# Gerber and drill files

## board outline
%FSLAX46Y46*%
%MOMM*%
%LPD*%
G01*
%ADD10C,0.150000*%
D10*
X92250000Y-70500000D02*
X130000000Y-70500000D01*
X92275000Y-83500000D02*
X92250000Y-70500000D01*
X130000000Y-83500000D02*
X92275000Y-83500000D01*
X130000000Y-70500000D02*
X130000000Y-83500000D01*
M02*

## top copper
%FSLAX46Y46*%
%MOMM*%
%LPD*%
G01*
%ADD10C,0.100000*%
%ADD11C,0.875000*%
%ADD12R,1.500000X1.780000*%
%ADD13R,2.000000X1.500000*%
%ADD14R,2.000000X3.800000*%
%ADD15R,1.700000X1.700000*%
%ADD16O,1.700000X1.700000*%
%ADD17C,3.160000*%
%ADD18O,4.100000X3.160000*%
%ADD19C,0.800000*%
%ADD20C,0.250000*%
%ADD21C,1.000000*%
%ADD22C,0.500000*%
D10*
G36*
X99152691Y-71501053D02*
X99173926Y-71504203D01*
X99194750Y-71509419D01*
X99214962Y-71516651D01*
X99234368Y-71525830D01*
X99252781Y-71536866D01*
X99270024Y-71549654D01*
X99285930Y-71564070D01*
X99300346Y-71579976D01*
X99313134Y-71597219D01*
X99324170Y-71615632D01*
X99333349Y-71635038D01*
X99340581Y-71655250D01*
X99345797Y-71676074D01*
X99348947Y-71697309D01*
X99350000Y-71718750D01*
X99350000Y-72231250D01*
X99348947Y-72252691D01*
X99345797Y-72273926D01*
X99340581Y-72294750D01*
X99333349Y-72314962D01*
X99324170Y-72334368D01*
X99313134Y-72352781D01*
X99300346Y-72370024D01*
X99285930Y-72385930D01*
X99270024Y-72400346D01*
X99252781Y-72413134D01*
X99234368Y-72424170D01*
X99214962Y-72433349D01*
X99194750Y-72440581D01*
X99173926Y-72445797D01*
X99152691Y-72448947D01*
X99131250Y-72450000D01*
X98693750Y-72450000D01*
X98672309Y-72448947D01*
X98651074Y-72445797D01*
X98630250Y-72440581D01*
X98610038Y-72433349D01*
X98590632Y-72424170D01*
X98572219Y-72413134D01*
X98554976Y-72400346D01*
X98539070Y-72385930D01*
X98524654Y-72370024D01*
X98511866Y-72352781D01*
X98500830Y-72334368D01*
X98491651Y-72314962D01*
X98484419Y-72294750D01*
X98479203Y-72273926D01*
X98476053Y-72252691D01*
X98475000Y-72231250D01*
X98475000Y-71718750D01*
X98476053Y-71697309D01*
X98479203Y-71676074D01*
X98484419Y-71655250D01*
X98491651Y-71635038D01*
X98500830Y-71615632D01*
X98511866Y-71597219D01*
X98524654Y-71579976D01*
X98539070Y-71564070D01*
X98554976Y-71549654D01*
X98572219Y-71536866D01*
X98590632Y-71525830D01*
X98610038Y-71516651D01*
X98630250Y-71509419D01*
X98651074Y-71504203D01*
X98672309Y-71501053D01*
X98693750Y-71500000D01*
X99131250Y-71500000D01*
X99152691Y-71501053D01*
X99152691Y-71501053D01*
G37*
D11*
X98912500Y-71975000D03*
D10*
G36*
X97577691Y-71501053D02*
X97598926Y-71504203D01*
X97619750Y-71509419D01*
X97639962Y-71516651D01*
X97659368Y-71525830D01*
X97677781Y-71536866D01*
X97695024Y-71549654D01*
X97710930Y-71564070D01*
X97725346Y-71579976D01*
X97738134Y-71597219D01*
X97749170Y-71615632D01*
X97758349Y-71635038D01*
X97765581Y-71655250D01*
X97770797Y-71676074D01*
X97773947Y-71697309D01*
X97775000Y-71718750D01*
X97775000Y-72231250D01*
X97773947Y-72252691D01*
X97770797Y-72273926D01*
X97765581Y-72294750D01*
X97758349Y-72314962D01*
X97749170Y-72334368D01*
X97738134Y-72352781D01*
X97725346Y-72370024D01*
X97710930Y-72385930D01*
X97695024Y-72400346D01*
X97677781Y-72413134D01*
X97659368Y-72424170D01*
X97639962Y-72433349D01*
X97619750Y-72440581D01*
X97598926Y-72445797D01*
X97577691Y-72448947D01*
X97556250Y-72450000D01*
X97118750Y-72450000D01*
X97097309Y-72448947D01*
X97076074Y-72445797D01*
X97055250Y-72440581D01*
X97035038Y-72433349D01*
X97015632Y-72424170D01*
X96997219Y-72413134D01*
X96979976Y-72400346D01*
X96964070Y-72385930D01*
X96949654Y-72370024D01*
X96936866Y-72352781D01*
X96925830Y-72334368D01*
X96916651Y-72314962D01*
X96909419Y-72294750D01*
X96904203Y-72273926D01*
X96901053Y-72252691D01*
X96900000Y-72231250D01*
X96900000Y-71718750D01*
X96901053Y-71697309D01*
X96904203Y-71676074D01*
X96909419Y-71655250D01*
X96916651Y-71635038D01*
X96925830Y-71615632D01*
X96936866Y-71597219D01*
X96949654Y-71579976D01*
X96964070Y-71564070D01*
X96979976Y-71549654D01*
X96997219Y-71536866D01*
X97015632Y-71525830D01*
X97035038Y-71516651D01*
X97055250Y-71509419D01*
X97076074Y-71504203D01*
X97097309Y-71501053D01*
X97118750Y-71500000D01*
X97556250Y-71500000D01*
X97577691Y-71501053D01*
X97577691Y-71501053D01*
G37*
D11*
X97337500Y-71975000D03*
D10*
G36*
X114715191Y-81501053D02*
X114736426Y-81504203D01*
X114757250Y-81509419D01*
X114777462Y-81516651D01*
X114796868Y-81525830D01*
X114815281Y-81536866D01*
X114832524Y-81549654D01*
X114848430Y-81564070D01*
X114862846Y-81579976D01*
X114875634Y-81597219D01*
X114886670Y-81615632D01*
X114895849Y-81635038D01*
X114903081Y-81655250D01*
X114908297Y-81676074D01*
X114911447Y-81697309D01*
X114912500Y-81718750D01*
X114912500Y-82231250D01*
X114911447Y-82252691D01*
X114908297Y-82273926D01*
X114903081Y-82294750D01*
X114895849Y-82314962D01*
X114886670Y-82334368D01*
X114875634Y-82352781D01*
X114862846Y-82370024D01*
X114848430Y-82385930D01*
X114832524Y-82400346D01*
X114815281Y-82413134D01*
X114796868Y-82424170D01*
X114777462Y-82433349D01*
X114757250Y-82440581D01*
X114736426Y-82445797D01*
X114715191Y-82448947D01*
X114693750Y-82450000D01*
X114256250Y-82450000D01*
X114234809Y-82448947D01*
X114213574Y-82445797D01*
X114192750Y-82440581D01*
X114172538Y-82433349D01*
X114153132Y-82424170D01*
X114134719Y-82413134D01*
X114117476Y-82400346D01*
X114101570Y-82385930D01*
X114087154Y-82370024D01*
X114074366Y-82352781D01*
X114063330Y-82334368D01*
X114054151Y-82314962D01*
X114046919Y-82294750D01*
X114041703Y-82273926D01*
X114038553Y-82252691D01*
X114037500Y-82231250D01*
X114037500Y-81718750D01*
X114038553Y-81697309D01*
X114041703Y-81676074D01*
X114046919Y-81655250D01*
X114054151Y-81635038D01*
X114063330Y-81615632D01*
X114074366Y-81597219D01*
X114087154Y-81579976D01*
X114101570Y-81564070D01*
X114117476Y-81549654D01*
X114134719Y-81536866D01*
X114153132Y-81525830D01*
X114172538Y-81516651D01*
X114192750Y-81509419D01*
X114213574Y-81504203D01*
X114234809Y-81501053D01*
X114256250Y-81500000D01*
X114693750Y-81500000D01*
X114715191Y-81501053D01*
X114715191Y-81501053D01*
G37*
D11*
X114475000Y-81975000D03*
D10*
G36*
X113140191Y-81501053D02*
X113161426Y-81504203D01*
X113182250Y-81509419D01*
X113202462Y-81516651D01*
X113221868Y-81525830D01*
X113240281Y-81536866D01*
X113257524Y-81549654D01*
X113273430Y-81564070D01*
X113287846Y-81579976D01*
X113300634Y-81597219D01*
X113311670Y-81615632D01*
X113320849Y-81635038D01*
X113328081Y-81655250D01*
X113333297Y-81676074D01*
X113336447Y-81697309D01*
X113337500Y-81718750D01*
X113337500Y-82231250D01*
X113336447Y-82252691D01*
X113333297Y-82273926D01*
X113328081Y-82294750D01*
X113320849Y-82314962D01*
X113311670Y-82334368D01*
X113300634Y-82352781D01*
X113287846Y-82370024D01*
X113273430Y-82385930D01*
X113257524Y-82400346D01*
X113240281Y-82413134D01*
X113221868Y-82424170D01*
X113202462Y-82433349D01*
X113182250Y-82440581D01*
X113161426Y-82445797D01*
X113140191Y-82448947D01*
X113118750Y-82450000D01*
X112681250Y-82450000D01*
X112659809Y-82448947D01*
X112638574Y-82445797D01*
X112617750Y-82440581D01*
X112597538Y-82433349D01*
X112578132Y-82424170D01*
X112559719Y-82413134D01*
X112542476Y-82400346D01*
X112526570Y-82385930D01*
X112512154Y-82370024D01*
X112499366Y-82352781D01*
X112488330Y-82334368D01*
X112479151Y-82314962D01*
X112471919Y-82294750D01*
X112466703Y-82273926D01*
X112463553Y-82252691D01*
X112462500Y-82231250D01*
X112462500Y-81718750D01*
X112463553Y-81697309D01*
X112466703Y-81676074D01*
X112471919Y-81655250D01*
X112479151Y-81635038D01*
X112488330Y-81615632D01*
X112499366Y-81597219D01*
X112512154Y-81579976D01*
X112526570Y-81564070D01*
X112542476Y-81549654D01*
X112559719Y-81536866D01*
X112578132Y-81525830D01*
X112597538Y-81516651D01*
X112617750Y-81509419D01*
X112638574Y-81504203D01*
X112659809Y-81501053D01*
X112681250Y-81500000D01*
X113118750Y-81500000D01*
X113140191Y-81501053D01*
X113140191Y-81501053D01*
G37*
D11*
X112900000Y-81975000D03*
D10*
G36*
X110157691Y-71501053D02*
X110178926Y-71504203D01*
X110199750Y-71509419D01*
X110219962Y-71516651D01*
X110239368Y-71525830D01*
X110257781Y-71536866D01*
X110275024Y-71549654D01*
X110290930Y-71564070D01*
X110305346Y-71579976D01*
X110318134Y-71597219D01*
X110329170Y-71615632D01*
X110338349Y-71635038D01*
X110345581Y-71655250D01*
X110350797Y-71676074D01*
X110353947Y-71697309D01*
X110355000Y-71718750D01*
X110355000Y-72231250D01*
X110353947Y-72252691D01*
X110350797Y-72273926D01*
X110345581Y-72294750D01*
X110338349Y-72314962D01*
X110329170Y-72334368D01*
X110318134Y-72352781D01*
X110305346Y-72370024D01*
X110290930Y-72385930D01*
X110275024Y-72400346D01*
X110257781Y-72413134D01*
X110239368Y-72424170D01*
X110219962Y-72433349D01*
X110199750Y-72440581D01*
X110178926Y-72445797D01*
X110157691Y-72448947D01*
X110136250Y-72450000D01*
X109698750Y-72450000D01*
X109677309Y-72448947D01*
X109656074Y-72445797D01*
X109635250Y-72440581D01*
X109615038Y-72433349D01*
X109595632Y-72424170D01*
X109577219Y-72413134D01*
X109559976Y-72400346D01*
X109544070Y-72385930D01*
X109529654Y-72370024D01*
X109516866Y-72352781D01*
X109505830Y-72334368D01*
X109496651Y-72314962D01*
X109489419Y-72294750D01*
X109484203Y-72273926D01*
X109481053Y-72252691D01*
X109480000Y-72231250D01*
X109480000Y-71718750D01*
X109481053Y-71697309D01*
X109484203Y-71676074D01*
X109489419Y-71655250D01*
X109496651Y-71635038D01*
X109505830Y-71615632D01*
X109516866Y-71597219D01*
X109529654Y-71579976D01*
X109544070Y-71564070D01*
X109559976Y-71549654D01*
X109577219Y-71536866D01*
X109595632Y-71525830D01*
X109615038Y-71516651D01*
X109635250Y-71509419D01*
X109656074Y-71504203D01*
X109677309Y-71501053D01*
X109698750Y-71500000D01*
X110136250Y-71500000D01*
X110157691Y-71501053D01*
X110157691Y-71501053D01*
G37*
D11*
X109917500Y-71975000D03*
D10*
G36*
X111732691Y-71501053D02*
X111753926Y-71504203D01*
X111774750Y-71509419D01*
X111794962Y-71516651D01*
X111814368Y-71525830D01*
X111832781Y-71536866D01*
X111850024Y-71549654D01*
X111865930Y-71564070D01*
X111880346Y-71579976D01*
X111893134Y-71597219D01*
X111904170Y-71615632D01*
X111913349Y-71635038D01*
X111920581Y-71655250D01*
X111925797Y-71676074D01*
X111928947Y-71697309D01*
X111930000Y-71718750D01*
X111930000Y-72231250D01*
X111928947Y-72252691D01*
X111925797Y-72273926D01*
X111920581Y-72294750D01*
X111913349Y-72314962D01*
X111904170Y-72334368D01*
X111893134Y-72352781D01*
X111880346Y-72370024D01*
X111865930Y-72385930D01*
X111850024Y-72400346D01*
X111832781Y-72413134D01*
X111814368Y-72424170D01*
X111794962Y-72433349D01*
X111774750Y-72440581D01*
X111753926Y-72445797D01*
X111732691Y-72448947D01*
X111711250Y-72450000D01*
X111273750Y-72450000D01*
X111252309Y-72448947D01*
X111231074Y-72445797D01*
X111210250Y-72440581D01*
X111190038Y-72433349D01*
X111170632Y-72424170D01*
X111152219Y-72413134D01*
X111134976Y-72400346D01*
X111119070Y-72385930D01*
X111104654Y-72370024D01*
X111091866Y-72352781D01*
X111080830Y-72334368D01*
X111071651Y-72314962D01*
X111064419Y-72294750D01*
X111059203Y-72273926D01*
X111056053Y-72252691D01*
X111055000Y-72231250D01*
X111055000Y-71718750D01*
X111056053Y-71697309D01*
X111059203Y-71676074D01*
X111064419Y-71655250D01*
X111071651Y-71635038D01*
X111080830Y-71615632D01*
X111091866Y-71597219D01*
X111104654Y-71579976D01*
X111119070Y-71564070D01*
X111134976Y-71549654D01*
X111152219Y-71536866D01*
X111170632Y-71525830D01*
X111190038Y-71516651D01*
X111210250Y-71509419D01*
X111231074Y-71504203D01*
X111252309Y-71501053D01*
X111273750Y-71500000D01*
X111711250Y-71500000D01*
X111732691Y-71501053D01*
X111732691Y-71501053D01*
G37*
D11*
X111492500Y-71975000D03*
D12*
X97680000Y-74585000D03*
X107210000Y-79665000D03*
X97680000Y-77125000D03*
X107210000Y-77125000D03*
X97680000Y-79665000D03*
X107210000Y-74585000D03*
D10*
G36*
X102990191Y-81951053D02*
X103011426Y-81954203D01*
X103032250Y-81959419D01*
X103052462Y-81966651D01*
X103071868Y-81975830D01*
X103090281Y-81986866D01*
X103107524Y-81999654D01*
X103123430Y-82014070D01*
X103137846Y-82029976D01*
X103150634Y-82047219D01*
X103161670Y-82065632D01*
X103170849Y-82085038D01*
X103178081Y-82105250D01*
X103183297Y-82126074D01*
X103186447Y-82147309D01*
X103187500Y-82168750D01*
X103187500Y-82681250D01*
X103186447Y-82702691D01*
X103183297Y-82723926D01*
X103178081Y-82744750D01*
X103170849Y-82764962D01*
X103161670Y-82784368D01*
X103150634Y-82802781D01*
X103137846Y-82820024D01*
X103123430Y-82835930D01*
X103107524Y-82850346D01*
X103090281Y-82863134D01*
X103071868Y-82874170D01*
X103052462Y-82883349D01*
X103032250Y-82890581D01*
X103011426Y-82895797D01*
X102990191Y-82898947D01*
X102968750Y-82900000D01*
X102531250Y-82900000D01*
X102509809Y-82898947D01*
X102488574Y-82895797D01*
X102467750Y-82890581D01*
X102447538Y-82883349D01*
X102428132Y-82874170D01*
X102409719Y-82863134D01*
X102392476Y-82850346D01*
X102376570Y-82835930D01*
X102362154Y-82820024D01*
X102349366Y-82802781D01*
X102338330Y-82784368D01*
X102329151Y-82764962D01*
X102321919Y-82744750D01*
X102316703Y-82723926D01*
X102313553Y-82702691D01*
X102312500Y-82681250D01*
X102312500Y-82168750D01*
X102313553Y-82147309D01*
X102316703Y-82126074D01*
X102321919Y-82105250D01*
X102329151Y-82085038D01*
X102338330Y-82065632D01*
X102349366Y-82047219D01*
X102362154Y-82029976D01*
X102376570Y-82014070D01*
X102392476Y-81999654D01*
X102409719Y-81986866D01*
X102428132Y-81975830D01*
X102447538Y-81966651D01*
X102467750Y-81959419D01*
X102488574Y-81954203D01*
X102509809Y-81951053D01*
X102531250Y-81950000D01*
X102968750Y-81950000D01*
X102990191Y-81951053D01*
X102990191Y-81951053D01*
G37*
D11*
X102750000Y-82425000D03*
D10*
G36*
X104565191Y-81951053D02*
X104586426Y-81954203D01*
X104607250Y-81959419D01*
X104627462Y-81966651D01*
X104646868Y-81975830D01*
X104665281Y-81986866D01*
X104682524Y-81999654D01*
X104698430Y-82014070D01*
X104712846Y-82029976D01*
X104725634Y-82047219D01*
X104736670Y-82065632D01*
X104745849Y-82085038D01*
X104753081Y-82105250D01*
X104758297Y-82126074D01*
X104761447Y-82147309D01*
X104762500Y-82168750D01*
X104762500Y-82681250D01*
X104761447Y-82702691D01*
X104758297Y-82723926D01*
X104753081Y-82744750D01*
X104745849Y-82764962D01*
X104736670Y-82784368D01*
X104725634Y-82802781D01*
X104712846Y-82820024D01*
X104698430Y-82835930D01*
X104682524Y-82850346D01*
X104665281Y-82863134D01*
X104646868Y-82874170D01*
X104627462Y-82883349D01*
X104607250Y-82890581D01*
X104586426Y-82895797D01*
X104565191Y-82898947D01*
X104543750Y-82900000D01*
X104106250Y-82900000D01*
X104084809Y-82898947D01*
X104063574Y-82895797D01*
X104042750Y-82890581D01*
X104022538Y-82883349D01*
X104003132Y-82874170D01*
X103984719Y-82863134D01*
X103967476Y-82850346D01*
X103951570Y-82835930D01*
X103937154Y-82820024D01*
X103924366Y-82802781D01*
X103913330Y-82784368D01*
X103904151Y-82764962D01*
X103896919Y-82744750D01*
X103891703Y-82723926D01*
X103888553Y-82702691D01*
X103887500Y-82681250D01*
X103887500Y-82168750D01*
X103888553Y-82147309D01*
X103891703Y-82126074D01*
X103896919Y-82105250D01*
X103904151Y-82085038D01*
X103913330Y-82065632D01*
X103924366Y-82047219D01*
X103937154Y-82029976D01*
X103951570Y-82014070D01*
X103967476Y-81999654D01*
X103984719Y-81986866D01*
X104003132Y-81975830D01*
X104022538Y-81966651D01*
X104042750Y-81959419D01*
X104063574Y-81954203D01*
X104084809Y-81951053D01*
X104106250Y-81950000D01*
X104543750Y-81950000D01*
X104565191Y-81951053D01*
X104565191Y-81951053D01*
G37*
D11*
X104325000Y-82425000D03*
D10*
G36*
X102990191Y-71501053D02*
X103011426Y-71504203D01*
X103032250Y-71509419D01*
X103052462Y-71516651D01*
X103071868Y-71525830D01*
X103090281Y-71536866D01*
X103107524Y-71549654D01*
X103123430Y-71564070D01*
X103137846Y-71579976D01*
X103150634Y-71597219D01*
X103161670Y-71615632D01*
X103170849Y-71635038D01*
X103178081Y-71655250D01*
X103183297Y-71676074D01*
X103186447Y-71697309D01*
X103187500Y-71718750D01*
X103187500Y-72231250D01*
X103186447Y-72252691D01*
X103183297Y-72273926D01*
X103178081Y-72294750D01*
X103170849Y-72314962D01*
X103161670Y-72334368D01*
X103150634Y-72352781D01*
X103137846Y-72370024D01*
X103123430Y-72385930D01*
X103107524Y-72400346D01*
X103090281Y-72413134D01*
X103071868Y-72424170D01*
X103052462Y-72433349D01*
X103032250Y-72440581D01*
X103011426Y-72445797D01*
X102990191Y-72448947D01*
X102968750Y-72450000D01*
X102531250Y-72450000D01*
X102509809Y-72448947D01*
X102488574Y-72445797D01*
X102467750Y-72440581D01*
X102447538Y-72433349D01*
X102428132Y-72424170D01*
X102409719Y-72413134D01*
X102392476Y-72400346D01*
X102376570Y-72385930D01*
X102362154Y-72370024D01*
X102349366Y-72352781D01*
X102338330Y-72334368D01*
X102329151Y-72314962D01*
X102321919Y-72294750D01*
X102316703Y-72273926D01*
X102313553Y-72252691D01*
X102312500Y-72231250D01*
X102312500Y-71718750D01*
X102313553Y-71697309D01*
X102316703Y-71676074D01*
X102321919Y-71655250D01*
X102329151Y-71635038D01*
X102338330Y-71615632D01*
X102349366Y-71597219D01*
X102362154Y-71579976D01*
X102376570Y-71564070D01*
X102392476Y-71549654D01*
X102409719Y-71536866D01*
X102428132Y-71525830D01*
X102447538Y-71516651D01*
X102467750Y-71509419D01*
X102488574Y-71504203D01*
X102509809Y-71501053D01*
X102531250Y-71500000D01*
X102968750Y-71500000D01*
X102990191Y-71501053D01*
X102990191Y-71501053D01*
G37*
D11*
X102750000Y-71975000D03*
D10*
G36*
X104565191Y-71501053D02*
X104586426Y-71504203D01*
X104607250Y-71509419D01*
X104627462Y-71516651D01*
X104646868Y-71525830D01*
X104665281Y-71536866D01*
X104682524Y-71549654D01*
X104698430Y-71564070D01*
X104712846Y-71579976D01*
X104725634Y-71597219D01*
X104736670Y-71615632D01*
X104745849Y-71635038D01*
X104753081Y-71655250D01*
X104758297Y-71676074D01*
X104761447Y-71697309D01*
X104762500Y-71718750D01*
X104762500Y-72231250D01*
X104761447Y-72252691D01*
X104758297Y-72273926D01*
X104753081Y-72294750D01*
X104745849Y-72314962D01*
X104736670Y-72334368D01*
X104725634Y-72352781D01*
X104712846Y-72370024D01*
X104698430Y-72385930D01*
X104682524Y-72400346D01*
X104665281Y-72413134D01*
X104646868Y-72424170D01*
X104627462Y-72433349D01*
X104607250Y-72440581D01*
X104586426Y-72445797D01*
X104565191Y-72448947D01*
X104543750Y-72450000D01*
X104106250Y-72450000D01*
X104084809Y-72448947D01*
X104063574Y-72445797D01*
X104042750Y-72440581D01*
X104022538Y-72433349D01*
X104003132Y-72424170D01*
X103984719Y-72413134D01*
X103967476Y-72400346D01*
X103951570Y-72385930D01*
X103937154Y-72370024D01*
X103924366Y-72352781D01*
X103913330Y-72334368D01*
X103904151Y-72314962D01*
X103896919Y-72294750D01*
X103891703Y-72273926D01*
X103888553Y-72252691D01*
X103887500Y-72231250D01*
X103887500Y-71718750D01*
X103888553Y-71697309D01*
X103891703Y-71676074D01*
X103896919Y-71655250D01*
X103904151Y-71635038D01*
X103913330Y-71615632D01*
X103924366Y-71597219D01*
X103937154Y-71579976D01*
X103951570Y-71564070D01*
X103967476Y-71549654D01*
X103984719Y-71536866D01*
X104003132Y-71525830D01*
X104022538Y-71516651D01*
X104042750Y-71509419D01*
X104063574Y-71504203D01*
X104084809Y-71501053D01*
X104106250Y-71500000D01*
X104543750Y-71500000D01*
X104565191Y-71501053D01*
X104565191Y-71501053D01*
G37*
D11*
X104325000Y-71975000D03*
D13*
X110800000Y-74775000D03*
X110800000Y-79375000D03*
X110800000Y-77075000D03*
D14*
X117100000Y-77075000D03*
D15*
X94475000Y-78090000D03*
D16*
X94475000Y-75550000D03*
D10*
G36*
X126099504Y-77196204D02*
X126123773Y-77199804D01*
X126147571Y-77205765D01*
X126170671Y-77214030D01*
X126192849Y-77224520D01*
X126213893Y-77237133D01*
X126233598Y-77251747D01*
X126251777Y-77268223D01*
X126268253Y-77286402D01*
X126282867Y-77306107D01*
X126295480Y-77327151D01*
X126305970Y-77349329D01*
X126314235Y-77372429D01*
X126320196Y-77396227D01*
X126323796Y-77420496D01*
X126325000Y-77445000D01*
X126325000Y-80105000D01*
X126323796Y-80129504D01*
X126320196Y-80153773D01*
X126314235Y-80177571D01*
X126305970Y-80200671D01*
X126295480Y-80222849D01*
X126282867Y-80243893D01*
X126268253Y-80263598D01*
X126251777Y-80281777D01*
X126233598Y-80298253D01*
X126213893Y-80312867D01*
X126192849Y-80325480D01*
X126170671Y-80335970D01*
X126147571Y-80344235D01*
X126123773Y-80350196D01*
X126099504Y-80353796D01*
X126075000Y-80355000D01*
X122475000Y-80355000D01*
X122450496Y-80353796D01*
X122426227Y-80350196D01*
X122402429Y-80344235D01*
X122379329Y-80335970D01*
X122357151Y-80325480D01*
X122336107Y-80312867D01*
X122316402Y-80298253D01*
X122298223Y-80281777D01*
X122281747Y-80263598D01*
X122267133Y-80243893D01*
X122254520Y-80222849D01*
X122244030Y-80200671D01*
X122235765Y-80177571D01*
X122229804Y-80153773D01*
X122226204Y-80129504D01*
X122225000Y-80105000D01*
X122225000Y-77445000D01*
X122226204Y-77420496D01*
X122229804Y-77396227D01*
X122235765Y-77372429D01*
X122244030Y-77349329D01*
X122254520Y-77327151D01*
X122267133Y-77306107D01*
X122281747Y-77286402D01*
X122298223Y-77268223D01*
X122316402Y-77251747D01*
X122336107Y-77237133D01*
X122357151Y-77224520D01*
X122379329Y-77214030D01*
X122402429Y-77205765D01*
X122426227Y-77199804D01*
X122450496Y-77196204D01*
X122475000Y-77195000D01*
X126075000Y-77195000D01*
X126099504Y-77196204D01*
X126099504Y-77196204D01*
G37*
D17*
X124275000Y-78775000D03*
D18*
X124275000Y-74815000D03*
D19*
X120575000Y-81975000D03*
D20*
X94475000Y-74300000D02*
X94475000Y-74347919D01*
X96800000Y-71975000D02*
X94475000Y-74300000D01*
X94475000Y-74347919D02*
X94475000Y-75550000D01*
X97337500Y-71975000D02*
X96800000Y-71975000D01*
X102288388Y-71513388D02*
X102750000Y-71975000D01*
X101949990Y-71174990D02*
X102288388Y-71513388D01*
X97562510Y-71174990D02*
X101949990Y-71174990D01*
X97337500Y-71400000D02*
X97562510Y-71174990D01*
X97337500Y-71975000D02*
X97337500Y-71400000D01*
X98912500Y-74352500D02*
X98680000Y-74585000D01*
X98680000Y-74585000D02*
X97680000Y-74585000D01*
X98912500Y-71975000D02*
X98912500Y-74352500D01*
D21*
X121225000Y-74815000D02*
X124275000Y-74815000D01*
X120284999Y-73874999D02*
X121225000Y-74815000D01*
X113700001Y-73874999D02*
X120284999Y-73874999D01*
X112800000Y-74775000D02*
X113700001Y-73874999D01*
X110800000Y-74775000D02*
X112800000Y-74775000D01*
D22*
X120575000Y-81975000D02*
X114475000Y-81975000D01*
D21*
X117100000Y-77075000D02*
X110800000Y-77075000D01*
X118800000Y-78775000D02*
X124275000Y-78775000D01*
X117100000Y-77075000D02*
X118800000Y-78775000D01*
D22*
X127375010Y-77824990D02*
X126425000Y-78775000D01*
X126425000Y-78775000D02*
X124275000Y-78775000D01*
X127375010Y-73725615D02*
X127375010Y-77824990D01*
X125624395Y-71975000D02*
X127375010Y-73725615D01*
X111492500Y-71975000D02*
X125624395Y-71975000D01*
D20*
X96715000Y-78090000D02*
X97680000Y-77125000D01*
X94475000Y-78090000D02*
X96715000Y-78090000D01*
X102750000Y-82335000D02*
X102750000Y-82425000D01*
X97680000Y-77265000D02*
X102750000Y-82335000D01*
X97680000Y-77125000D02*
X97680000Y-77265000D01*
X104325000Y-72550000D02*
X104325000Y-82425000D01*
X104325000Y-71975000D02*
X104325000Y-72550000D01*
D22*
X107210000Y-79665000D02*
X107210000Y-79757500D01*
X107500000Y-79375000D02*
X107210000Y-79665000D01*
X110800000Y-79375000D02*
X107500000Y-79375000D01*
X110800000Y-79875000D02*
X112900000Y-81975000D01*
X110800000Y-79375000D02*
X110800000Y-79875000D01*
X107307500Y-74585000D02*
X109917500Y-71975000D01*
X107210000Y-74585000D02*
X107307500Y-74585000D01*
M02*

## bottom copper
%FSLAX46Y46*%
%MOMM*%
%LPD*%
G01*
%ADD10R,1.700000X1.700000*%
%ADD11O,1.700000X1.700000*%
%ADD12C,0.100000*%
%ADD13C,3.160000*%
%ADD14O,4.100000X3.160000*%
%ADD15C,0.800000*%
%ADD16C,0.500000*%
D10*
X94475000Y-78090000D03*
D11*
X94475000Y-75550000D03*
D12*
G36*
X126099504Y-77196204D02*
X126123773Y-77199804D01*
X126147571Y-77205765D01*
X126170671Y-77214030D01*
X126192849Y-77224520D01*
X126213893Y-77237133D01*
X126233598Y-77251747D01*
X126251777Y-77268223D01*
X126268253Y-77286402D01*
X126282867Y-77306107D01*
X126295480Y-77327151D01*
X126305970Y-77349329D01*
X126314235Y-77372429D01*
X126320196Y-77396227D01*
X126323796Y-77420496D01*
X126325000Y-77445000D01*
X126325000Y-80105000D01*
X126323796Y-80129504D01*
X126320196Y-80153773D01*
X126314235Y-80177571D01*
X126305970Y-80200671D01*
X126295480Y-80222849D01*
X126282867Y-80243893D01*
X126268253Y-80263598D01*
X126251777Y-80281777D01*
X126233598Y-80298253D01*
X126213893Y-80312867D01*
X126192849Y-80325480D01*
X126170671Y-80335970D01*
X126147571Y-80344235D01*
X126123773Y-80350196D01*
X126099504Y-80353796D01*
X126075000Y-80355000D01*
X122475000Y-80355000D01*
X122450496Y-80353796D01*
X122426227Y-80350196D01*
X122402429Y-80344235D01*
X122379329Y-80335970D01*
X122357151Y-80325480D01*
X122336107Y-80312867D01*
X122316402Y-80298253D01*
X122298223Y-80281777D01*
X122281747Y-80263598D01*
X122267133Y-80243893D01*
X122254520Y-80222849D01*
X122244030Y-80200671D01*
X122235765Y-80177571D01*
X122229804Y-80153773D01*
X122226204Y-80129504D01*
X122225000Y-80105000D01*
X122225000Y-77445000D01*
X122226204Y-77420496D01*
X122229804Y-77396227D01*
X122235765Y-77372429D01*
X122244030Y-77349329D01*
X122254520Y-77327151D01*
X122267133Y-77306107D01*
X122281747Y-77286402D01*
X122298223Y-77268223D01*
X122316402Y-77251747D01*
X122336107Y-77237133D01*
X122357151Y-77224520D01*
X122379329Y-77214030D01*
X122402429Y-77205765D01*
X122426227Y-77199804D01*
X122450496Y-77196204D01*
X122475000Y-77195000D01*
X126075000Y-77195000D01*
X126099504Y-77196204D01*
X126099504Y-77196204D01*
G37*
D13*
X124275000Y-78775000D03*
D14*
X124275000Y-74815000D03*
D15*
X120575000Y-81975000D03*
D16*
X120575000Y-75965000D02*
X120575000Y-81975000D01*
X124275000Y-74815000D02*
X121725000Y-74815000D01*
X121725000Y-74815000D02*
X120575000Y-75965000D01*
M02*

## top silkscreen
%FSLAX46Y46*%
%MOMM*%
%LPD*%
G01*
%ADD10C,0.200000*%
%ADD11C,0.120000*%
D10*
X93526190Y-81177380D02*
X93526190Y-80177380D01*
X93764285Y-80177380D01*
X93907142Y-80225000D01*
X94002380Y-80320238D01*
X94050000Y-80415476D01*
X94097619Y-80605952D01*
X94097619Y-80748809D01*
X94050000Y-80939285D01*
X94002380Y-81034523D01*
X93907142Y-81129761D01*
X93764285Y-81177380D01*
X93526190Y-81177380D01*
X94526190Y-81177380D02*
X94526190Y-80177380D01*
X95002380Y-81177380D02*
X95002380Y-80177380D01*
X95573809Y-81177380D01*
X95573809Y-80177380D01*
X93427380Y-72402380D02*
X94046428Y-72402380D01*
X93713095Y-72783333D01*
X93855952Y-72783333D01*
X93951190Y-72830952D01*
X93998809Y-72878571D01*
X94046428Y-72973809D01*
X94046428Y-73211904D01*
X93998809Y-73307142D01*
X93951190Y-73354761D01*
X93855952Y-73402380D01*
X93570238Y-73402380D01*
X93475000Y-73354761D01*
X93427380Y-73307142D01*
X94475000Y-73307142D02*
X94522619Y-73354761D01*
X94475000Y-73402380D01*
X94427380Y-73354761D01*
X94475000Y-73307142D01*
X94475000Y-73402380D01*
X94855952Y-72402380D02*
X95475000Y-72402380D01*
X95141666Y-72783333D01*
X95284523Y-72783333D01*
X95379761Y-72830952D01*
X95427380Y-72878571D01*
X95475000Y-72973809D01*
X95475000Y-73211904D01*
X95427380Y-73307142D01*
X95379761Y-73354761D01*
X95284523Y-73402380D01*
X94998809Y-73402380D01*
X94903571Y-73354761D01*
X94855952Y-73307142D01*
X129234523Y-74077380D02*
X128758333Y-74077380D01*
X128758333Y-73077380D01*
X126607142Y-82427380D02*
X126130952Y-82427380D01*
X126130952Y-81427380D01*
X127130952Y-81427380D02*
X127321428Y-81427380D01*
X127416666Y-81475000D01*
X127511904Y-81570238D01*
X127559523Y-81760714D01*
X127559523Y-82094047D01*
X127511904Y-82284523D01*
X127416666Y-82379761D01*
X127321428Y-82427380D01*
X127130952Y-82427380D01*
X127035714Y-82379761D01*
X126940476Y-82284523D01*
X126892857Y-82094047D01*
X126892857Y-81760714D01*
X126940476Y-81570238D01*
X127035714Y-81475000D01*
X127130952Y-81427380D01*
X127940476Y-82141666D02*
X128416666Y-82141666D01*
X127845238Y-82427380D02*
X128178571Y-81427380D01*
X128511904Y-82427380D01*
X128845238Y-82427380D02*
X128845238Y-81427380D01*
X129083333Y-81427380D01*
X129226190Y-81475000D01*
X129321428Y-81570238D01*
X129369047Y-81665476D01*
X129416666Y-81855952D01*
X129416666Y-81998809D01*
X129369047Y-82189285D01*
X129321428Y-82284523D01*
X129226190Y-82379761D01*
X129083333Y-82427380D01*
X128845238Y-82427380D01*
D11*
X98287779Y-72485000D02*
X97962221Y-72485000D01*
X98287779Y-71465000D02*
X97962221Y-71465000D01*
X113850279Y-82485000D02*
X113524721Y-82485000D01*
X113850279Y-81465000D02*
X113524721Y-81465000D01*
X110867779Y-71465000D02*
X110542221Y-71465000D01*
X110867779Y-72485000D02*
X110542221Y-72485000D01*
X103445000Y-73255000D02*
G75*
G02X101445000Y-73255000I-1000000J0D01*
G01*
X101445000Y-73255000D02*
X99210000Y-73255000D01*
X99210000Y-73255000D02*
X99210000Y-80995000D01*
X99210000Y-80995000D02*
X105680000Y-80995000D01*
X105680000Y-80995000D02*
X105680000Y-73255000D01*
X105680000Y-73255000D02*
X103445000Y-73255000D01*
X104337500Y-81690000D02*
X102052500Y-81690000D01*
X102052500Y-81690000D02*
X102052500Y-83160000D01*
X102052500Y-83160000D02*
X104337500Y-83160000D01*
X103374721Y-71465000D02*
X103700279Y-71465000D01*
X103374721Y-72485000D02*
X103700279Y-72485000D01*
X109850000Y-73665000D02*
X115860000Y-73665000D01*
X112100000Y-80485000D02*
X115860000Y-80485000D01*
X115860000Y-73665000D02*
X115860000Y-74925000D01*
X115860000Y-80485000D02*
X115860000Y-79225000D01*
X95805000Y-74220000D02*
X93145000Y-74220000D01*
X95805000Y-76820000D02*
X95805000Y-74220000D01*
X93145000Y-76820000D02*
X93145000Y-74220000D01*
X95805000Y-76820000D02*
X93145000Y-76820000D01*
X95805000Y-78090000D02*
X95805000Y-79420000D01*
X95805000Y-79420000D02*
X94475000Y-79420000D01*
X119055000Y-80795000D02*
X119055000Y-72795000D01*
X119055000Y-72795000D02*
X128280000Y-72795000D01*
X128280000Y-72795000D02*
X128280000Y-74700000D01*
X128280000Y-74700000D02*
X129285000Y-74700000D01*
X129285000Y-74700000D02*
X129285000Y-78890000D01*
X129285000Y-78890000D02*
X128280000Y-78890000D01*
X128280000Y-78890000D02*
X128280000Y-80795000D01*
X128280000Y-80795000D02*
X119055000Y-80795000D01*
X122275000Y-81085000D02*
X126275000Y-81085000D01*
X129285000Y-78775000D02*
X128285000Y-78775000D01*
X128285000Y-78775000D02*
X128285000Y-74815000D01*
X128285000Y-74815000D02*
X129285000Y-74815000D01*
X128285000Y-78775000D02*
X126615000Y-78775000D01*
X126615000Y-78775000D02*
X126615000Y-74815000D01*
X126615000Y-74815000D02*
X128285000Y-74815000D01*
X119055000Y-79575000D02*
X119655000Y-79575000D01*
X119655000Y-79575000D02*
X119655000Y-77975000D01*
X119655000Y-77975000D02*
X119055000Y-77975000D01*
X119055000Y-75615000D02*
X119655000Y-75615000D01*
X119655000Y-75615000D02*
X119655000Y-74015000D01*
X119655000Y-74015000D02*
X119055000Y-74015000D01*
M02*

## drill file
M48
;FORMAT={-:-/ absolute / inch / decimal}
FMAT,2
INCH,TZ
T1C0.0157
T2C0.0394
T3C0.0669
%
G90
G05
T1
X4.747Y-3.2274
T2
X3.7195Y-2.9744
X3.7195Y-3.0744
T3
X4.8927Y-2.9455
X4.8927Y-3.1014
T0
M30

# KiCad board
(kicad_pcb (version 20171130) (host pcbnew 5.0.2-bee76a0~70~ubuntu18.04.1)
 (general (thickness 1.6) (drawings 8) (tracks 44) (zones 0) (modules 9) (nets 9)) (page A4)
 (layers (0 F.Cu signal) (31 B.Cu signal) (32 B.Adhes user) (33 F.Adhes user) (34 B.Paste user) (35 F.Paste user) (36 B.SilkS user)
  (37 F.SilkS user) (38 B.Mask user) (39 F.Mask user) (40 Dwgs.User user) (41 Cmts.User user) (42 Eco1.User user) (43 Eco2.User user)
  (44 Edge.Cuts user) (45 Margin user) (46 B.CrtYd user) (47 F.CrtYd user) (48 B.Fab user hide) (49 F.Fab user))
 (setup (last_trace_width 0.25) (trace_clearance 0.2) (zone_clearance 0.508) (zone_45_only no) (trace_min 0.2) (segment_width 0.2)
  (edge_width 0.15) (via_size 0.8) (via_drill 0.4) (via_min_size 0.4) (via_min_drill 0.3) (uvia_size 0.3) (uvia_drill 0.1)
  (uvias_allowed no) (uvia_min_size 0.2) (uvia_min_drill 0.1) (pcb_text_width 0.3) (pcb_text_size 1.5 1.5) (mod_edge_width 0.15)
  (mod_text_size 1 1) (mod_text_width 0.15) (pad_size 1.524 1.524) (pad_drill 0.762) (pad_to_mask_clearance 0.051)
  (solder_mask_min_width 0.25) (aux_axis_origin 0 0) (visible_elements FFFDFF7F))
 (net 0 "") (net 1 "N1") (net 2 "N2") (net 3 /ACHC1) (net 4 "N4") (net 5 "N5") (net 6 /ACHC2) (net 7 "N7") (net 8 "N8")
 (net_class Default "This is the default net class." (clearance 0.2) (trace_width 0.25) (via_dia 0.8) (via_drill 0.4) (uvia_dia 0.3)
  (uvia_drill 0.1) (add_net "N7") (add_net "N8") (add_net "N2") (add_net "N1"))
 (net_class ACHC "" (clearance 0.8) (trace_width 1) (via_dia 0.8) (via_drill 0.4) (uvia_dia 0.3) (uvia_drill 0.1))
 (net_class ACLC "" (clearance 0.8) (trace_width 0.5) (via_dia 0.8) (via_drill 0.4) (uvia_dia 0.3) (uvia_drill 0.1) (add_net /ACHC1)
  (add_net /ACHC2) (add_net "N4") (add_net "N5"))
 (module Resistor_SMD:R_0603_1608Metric (layer F.Cu) (at 98.125 71.975 180)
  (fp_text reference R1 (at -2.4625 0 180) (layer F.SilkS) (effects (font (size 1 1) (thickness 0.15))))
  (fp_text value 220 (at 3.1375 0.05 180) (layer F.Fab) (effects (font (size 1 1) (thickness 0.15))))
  (fp_line (start -0.162779 -0.51) (end 0.162779 -0.51) (layer F.SilkS) (width 0.12))
  (fp_line (start -0.162779 0.51) (end 0.162779 0.51) (layer F.SilkS) (width 0.12))
  (pad 1 smd roundrect (at -0.7875 0 180) (size 0.875 0.95) (layers F.Cu F.Paste F.Mask) (roundrect_rratio 0.25) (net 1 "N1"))
  (pad 2 smd roundrect (at 0.7875 0 180) (size 0.875 0.95) (layers F.Cu F.Paste F.Mask) (roundrect_rratio 0.25) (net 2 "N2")))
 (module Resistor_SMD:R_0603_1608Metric (layer F.Cu) (at 113.6875 81.975 180)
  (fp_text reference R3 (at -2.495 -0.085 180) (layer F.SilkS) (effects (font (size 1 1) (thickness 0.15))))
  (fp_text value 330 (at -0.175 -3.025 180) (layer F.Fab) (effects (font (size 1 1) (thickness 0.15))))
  (fp_line (start -0.162779 -0.51) (end 0.162779 -0.51) (layer F.SilkS) (width 0.12))
  (fp_line (start -0.162779 0.51) (end 0.162779 0.51) (layer F.SilkS) (width 0.12))
  (pad 1 smd roundrect (at -0.7875 0 180) (size 0.875 0.95) (layers F.Cu F.Paste F.Mask) (roundrect_rratio 0.25) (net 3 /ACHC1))
  (pad 2 smd roundrect (at 0.7875 0 180) (size 0.875 0.95) (layers F.Cu F.Paste F.Mask) (roundrect_rratio 0.25) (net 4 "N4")))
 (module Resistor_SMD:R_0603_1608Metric (layer F.Cu) (at 110.705 71.975 180)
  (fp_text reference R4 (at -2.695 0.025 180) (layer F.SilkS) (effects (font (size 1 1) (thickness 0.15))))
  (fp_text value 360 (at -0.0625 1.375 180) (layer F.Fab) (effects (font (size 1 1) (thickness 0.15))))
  (fp_line (start -0.162779 0.51) (end 0.162779 0.51) (layer F.SilkS) (width 0.12))
  (fp_line (start -0.162779 -0.51) (end 0.162779 -0.51) (layer F.SilkS) (width 0.12))
  (pad 2 smd roundrect (at 0.7875 0 180) (size 0.875 0.95) (layers F.Cu F.Paste F.Mask) (roundrect_rratio 0.25) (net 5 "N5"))
  (pad 1 smd roundrect (at -0.7875 0 180) (size 0.875 0.95) (layers F.Cu F.Paste F.Mask) (roundrect_rratio 0.25) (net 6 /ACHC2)))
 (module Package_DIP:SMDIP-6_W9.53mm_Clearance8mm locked (layer F.Cu) (at 102.445 77.125)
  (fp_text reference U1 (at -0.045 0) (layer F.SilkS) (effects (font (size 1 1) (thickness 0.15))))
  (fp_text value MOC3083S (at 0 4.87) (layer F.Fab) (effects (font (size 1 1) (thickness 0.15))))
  (fp_arc (start 0 -3.87) (end -1 -3.87) (angle -180) (layer F.SilkS) (width 0.12))
  (fp_line (start -1 -3.87) (end -3.235 -3.87) (layer F.SilkS) (width 0.12))
  (fp_line (start -3.235 -3.87) (end -3.235 3.87) (layer F.SilkS) (width 0.12))
  (fp_line (start -3.235 3.87) (end 3.235 3.87) (layer F.SilkS) (width 0.12))
  (fp_line (start 3.235 3.87) (end 3.235 -3.87) (layer F.SilkS) (width 0.12))
  (fp_line (start 3.235 -3.87) (end 1 -3.87) (layer F.SilkS) (width 0.12))
  (pad 1 smd rect (at -4.765 -2.54) (size 1.5 1.78) (layers F.Cu F.Paste F.Mask) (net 1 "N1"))
  (pad 4 smd rect (at 4.765 2.54) (size 1.5 1.78) (layers F.Cu F.Paste F.Mask) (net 4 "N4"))
  (pad 2 smd rect (at -4.765 0) (size 1.5 1.78) (layers F.Cu F.Paste F.Mask) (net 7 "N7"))
  (pad 5 smd rect (at 4.765 0) (size 1.5 1.78) (layers F.Cu F.Paste F.Mask))
  (pad 3 smd rect (at -4.765 2.54) (size 1.5 1.78) (layers F.Cu F.Paste F.Mask))
  (pad 6 smd rect (at 4.765 -2.54) (size 1.5 1.78) (layers F.Cu F.Paste F.Mask) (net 5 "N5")))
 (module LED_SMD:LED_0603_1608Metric (layer F.Cu) (at 103.5375 82.425)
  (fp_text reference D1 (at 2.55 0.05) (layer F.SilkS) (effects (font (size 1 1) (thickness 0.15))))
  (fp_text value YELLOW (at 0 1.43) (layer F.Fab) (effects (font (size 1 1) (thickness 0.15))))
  (fp_line (start 0.8 -0.735) (end -1.485 -0.735) (layer F.SilkS) (width 0.12))
  (fp_line (start -1.485 -0.735) (end -1.485 0.735) (layer F.SilkS) (width 0.12))
  (fp_line (start -1.485 0.735) (end 0.8 0.735) (layer F.SilkS) (width 0.12))
  (pad 1 smd roundrect (at -0.7875 0) (size 0.875 0.95) (layers F.Cu F.Paste F.Mask) (roundrect_rratio 0.25) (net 7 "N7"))
  (pad 2 smd roundrect (at 0.7875 0) (size 0.875 0.95) (layers F.Cu F.Paste F.Mask) (roundrect_rratio 0.25) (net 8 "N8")))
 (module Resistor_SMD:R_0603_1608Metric (layer F.Cu) (at 103.5375 71.975)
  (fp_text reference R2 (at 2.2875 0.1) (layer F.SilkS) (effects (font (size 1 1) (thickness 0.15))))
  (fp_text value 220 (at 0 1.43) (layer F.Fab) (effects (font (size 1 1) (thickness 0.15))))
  (fp_line (start -0.162779 -0.51) (end 0.162779 -0.51) (layer F.SilkS) (width 0.12))
  (fp_line (start -0.162779 0.51) (end 0.162779 0.51) (layer F.SilkS) (width 0.12))
  (pad 1 smd roundrect (at -0.7875 0) (size 0.875 0.95) (layers F.Cu F.Paste F.Mask) (roundrect_rratio 0.25) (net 2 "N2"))
  (pad 2 smd roundrect (at 0.7875 0) (size 0.875 0.95) (layers F.Cu F.Paste F.Mask) (roundrect_rratio 0.25) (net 8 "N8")))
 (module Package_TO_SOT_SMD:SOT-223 (layer F.Cu) (at 113.95 77.075)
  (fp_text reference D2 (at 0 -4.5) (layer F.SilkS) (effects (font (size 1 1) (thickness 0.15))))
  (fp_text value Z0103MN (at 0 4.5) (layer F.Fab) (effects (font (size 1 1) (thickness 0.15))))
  (fp_line (start -4.1 -3.41) (end 1.91 -3.41) (layer F.SilkS) (width 0.12))
  (fp_line (start -1.85 3.41) (end 1.91 3.41) (layer F.SilkS) (width 0.12))
  (fp_line (start 1.91 -3.41) (end 1.91 -2.15) (layer F.SilkS) (width 0.12))
  (fp_line (start 1.91 3.41) (end 1.91 2.15) (layer F.SilkS) (width 0.12))
  (pad 1 smd rect (at -3.15 -2.3) (size 2 1.5) (layers F.Cu F.Paste F.Mask) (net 3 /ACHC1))
  (pad 3 smd rect (at -3.15 2.3) (size 2 1.5) (layers F.Cu F.Paste F.Mask) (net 4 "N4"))
  (pad 2 smd rect (at -3.15 0) (size 2 1.5) (layers F.Cu F.Paste F.Mask) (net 6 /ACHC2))
  (pad 4 smd rect (at 3.15 0) (size 2 3.8) (layers F.Cu F.Paste F.Mask) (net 6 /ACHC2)))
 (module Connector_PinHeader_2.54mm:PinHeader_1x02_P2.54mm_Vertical (layer F.Cu) (at 94.475 78.09 180)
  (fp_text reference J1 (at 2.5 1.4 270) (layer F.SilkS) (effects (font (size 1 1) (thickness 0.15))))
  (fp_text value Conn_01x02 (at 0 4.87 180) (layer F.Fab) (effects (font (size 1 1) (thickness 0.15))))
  (fp_line (start -1.33 3.87) (end 1.33 3.87) (layer F.SilkS) (width 0.12))
  (fp_line (start -1.33 1.27) (end -1.33 3.87) (layer F.SilkS) (width 0.12))
  (fp_line (start 1.33 1.27) (end 1.33 3.87) (layer F.SilkS) (width 0.12))
  (fp_line (start -1.33 1.27) (end 1.33 1.27) (layer F.SilkS) (width 0.12))
  (fp_line (start -1.33 0) (end -1.33 -1.33) (layer F.SilkS) (width 0.12))
  (fp_line (start -1.33 -1.33) (end 0 -1.33) (layer F.SilkS) (width 0.12))
  (pad 1 thru_hole rect (at 0 0 180) (size 1.7 1.7) (drill 1) (layers *.Cu *.Mask) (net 7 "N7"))
  (pad 2 thru_hole oval (at 0 2.54 180) (size 1.7 1.7) (drill 1) (layers *.Cu *.Mask) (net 2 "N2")))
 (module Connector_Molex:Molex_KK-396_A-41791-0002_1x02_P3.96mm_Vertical (layer F.Cu) (at 124.275 78.775 90)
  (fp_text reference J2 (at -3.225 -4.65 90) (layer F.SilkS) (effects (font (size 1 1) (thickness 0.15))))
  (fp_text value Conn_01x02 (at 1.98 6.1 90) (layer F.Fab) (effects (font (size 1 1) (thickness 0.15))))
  (fp_line (start -2.02 -5.22) (end 5.98 -5.22) (layer F.SilkS) (width 0.12))
  (fp_line (start 5.98 -5.22) (end 5.98 4.005) (layer F.SilkS) (width 0.12))
  (fp_line (start 5.98 4.005) (end 4.075 4.005) (layer F.SilkS) (width 0.12))
  (fp_line (start 4.075 4.005) (end 4.075 5.01) (layer F.SilkS) (width 0.12))
  (fp_line (start 4.075 5.01) (end -0.115 5.01) (layer F.SilkS) (width 0.12))
  (fp_line (start -0.115 5.01) (end -0.115 4.005) (layer F.SilkS) (width 0.12))
  (fp_line (start -0.115 4.005) (end -2.02 4.005) (layer F.SilkS) (width 0.12))
  (fp_line (start -2.02 4.005) (end -2.02 -5.22) (layer F.SilkS) (width 0.12))
  (fp_line (start -2.31 -2) (end -2.31 2) (layer F.SilkS) (width 0.12))
  (fp_line (start 0 5.01) (end 0 4.01) (layer F.SilkS) (width 0.12))
  (fp_line (start 0 4.01) (end 3.96 4.01) (layer F.SilkS) (width 0.12))
  (fp_line (start 3.96 4.01) (end 3.96 5.01) (layer F.SilkS) (width 0.12))
  (fp_line (start 0 4.01) (end 0 2.34) (layer F.SilkS) (width 0.12))
  (fp_line (start 0 2.34) (end 3.96 2.34) (layer F.SilkS) (width 0.12))
  (fp_line (start 3.96 2.34) (end 3.96 4.01) (layer F.SilkS) (width 0.12))
  (fp_line (start -0.8 -5.22) (end -0.8 -4.62) (layer F.SilkS) (width 0.12))
  (fp_line (start -0.8 -4.62) (end 0.8 -4.62) (layer F.SilkS) (width 0.12))
  (fp_line (start 0.8 -4.62) (end 0.8 -5.22) (layer F.SilkS) (width 0.12))
  (fp_line (start 3.16 -5.22) (end 3.16 -4.62) (layer F.SilkS) (width 0.12))
  (fp_line (start 3.16 -4.62) (end 4.76 -4.62) (layer F.SilkS) (width 0.12))
  (fp_line (start 4.76 -4.62) (end 4.76 -5.22) (layer F.SilkS) (width 0.12))
  (pad 1 thru_hole roundrect (at 0 0 90) (size 3.16 4.1) (drill 1.7) (layers *.Cu *.Mask) (roundrect_rratio 0.079114) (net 6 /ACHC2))
  (pad 2 thru_hole oval (at 3.96 0 90) (size 3.16 4.1) (drill 1.7) (layers *.Cu *.Mask) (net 3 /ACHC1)))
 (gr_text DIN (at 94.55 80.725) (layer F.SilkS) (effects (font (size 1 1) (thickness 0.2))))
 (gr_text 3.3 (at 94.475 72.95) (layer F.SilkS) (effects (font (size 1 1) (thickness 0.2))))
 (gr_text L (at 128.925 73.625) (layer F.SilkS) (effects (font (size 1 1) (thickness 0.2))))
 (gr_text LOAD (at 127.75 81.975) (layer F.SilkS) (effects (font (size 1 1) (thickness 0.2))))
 (gr_line (start 92.25 70.5) (end 130 70.5) (layer Edge.Cuts) (width 0.15))
 (gr_line (start 92.275 83.5) (end 92.25 70.5) (layer Edge.Cuts) (width 0.15))
 (gr_line (start 130 83.5) (end 92.275 83.5) (layer Edge.Cuts) (width 0.15))
 (gr_line (start 130 70.5) (end 130 83.5) (layer Edge.Cuts) (width 0.15))
 (segment (start 94.475 74.3) (end 94.475 74.347919) (width 0.25) (layer F.Cu) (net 2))
 (segment (start 96.8 71.975) (end 94.475 74.3) (width 0.25) (layer F.Cu) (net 2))
 (segment (start 94.475 74.347919) (end 94.475 75.55) (width 0.25) (layer F.Cu) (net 2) (status 20))
 (segment (start 97.3375 71.975) (end 96.8 71.975) (width 0.25) (layer F.Cu) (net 2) (status 10))
 (segment (start 102.288388 71.513388) (end 102.75 71.975) (width 0.25) (layer F.Cu) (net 2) (status 20))
 (segment (start 101.94999 71.17499) (end 102.288388 71.513388) (width 0.25) (layer F.Cu) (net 2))
 (segment (start 97.56251 71.17499) (end 101.94999 71.17499) (width 0.25) (layer F.Cu) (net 2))
 (segment (start 97.3375 71.4) (end 97.56251 71.17499) (width 0.25) (layer F.Cu) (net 2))
 (segment (start 97.3375 71.975) (end 97.3375 71.4) (width 0.25) (layer F.Cu) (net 2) (status 10))
 (segment (start 98.9125 74.3525) (end 98.68 74.585) (width 0.25) (layer F.Cu) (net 1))
 (segment (start 98.68 74.585) (end 97.68 74.585) (width 0.25) (layer F.Cu) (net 1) (status 20))
 (segment (start 98.9125 71.975) (end 98.9125 74.3525) (width 0.25) (layer F.Cu) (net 1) (status 10))
 (segment (start 121.225 74.815) (end 124.275 74.815) (width 1) (layer F.Cu) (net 3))
 (segment (start 120.284999 73.874999) (end 121.225 74.815) (width 1) (layer F.Cu) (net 3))
 (segment (start 113.700001 73.874999) (end 120.284999 73.874999) (width 1) (layer F.Cu) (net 3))
 (segment (start 112.8 74.775) (end 113.700001 73.874999) (width 1) (layer F.Cu) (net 3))
 (segment (start 110.8 74.775) (end 112.8 74.775) (width 1) (layer F.Cu) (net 3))
 (segment (start 120.575 75.965) (end 120.575 81.975) (width 0.5) (layer B.Cu) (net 3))
 (via (at 120.575 81.975) (size 0.8) (drill 0.4) (layers F.Cu B.Cu) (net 3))
 (segment (start 124.275 74.815) (end 121.725 74.815) (width 0.5) (layer B.Cu) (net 3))
 (segment (start 121.725 74.815) (end 120.575 75.965) (width 0.5) (layer B.Cu) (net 3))
 (segment (start 120.575 81.975) (end 114.475 81.975) (width 0.5) (layer F.Cu) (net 3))
 (segment (start 117.1 77.075) (end 110.8 77.075) (width 1) (layer F.Cu) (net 6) (status 30))
 (segment (start 118.8 78.775) (end 124.275 78.775) (width 1) (layer F.Cu) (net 6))
 (segment (start 117.1 77.075) (end 118.8 78.775) (width 1) (layer F.Cu) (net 6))
 (segment (start 127.37501 77.82499) (end 126.425 78.775) (width 0.5) (layer F.Cu) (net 6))
 (segment (start 126.425 78.775) (end 124.275 78.775) (width 0.5) (layer F.Cu) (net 6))
 (segment (start 127.37501 73.725615) (end 127.37501 77.82499) (width 0.5) (layer F.Cu) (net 6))
 (segment (start 125.624395 71.975) (end 127.37501 73.725615) (width 0.5) (layer F.Cu) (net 6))
 (segment (start 111.4925 71.975) (end 125.624395 71.975) (width 0.5) (layer F.Cu) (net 6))
 (segment (start 96.715 78.09) (end 97.68 77.125) (width 0.25) (layer F.Cu) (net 7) (status 20))
 (segment (start 94.475 78.09) (end 96.715 78.09) (width 0.25) (layer F.Cu) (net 7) (status 10))
 (segment (start 102.75 82.335) (end 102.75 82.425) (width 0.25) (layer F.Cu) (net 7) (status 30))
 (segment (start 97.68 77.265) (end 102.75 82.335) (width 0.25) (layer F.Cu) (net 7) (status 30))
 (segment (start 97.68 77.125) (end 97.68 77.265) (width 0.25) (layer F.Cu) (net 7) (status 30))
 (segment (start 104.325 72.55) (end 104.325 82.425) (width 0.25) (layer F.Cu) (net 8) (status 20))
 (segment (start 104.325 71.975) (end 104.325 72.55) (width 0.25) (layer F.Cu) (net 8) (status 10))
 (segment (start 107.21 79.665) (end 107.21 79.7575) (width 0.5) (layer F.Cu) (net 4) (status 30))
 (segment (start 107.5 79.375) (end 107.21 79.665) (width 0.5) (layer F.Cu) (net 4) (status 30))
 (segment (start 110.8 79.375) (end 107.5 79.375) (width 0.5) (layer F.Cu) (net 4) (status 30))
 (segment (start 110.8 79.875) (end 112.9 81.975) (width 0.5) (layer F.Cu) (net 4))
 (segment (start 110.8 79.375) (end 110.8 79.875) (width 0.5) (layer F.Cu) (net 4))
 (segment (start 107.3075 74.585) (end 109.9175 71.975) (width 0.5) (layer F.Cu) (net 5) (status 30))
 (segment (start 107.21 74.585) (end 107.3075 74.585) (width 0.5) (layer F.Cu) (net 5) (status 30)))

